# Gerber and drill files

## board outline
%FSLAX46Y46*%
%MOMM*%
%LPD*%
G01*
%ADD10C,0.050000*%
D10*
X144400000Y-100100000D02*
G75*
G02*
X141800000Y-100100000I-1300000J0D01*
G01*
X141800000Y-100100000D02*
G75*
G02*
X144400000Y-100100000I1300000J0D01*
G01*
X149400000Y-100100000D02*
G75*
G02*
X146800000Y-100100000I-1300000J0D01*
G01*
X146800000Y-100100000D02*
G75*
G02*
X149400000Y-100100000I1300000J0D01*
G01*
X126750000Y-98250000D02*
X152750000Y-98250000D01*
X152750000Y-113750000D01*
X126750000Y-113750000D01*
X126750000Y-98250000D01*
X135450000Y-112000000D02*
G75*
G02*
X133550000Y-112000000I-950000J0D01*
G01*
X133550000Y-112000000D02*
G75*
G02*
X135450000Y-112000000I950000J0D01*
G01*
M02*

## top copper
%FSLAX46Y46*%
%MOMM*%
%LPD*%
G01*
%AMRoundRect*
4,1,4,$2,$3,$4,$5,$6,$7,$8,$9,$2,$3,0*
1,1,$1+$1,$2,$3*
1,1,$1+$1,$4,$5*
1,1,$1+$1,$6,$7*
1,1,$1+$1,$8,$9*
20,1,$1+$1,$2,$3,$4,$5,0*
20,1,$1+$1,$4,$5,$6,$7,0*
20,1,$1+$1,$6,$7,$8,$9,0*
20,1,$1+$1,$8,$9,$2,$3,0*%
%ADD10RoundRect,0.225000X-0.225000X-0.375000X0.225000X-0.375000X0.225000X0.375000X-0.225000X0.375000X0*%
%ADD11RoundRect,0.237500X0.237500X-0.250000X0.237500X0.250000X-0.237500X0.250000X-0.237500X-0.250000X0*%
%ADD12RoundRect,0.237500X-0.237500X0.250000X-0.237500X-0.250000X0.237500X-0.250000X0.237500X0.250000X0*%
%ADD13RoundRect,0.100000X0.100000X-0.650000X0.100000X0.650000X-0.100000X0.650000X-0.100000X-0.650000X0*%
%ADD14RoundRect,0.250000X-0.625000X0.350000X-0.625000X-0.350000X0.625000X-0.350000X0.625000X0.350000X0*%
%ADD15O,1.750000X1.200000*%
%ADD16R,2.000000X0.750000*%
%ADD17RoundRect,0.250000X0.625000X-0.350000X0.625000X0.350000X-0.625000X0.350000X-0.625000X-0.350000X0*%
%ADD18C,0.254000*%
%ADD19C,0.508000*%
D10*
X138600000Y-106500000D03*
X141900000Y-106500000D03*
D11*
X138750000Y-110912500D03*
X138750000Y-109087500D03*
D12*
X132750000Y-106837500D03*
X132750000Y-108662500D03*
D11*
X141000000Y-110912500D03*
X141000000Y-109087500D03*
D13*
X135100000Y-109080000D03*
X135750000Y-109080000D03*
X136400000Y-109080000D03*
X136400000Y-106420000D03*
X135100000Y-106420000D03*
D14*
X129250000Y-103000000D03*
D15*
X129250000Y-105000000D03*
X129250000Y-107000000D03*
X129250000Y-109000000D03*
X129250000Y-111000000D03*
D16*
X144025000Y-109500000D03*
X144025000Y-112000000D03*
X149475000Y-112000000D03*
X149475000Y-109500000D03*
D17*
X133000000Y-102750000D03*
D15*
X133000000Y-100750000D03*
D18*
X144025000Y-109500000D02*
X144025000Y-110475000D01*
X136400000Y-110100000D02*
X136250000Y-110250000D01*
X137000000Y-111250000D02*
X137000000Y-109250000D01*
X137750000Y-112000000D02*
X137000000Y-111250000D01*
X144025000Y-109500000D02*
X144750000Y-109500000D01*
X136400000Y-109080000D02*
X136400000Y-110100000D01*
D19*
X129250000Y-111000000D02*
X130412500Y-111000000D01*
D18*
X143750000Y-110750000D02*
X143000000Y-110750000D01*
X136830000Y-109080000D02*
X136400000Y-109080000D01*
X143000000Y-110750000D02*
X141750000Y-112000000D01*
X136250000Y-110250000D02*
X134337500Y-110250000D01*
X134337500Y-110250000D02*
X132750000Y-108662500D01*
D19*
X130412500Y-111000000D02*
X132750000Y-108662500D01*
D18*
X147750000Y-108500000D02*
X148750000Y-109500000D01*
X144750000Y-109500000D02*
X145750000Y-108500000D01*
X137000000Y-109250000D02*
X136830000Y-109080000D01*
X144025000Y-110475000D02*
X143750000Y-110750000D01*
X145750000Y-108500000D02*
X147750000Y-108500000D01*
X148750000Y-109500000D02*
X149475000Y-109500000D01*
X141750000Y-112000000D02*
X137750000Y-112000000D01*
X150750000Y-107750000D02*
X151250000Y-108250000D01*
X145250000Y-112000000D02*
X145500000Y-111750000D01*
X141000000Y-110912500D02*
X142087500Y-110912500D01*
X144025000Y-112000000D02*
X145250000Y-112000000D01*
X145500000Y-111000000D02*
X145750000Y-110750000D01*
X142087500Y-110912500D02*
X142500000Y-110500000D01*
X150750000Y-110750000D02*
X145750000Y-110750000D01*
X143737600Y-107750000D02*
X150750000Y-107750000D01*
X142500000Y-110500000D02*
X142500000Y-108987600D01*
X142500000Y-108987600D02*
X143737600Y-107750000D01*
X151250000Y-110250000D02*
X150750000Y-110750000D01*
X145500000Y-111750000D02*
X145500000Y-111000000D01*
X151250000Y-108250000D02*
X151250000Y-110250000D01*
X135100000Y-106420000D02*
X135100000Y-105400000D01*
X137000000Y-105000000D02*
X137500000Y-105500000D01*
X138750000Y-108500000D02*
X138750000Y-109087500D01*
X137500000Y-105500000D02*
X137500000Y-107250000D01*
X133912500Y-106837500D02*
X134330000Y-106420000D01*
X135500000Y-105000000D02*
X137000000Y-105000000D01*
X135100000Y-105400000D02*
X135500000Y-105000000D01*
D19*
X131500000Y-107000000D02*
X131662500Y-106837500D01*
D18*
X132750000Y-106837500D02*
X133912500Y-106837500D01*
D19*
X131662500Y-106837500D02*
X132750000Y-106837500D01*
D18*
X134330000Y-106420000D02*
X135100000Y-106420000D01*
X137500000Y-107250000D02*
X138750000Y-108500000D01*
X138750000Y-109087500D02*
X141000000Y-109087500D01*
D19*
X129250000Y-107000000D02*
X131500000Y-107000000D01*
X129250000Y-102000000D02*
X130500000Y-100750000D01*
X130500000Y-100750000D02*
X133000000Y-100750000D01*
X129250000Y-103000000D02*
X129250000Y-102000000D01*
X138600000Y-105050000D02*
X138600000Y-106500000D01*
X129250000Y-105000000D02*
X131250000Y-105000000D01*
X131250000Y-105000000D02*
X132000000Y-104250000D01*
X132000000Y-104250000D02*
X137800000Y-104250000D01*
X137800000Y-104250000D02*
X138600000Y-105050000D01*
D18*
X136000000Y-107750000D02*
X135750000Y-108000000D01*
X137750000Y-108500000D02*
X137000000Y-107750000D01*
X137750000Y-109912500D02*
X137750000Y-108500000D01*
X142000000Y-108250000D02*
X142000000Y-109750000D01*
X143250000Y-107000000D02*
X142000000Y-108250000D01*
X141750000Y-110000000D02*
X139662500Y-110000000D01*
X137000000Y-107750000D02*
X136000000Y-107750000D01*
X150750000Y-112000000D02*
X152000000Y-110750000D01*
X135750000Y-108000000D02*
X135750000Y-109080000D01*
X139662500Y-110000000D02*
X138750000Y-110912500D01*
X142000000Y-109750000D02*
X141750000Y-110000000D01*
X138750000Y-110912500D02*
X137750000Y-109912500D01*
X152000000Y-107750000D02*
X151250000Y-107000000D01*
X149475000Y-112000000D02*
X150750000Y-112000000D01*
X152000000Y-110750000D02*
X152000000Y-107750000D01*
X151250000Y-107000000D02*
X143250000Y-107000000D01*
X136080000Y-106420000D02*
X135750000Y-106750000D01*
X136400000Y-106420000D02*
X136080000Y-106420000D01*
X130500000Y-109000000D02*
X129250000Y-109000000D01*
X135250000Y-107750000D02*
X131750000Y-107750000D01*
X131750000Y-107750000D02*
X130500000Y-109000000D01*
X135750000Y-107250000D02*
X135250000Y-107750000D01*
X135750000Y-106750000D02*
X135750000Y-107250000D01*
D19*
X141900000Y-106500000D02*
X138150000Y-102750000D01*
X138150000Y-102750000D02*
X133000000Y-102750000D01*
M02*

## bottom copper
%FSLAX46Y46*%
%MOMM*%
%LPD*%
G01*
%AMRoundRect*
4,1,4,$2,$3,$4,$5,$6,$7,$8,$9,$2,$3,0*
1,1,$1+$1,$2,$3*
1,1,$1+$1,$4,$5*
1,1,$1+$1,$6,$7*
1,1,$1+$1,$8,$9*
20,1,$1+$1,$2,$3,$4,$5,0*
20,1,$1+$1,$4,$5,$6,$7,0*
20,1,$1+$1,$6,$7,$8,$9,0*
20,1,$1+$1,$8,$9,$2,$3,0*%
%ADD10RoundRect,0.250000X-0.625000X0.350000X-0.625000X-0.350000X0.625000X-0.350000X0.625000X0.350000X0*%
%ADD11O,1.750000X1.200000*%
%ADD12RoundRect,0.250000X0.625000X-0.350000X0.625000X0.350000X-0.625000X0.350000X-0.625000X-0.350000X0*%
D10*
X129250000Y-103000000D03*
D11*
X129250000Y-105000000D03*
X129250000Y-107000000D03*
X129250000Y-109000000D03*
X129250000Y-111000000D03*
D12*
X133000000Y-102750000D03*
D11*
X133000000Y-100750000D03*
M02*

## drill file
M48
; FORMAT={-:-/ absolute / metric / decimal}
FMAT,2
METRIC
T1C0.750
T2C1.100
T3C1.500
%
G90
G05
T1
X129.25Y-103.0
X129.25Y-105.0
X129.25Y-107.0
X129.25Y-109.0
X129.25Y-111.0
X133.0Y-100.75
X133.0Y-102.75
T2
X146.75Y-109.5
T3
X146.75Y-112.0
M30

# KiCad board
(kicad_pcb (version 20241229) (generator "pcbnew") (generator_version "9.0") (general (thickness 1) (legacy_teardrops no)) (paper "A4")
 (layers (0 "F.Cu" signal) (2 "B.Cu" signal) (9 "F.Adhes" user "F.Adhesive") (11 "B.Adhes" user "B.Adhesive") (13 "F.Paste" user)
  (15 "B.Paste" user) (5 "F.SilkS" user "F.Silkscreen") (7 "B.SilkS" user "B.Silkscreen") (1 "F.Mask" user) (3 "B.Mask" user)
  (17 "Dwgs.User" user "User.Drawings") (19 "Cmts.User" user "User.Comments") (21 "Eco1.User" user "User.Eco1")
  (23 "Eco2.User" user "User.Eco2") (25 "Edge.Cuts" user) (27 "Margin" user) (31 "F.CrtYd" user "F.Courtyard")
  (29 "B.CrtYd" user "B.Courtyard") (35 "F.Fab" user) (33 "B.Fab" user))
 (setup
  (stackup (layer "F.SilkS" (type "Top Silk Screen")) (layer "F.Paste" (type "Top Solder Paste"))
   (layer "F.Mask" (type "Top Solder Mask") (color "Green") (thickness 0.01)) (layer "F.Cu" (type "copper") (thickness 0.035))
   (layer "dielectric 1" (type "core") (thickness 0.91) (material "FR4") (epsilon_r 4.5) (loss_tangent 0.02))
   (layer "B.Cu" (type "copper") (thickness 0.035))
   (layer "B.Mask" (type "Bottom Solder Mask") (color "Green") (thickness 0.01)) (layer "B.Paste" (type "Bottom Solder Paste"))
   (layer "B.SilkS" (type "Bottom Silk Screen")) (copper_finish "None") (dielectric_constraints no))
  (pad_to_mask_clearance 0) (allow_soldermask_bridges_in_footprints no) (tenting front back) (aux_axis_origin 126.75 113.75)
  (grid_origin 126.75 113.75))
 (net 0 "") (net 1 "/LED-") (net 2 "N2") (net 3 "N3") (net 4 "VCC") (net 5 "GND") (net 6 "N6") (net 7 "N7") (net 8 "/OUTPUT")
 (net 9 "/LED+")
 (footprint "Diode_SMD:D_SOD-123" (layer "F.Cu") (at 140.25 106.5)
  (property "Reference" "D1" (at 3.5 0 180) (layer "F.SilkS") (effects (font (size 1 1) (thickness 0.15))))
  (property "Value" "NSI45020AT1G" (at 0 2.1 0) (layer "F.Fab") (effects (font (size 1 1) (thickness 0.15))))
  (pad "1" smd roundrect (at -1.65 0) (size 0.9 1.2) (layers "F.Cu" "F.Mask" "F.Paste") (roundrect_rratio 0.25) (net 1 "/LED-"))
  (pad "2" smd roundrect (at 1.65 0) (size 0.9 1.2) (layers "F.Cu" "F.Mask" "F.Paste") (roundrect_rratio 0.25) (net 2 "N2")))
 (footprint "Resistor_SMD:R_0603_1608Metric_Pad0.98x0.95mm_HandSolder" (layer "F.Cu") (at 138.75 110 90)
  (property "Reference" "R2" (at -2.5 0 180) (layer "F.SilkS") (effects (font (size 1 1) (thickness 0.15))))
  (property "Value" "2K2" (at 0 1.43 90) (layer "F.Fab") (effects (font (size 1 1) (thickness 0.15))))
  (pad "1" smd roundrect (at -0.9125 0 90) (size 0.975 0.95) (layers "F.Cu" "F.Mask" "F.Paste") (roundrect_rratio 0.25) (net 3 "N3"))
  (pad "2" smd roundrect (at 0.9125 0 90) (size 0.975 0.95) (layers "F.Cu" "F.Mask" "F.Paste") (roundrect_rratio 0.25) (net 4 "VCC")))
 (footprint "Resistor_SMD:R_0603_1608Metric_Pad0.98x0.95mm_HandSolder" (layer "F.Cu") (at 132.75 107.75 -90)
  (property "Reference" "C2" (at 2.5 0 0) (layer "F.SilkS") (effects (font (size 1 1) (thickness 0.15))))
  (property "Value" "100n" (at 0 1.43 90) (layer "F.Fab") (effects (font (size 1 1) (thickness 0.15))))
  (pad "1" smd roundrect (at -0.9125 0 270) (size 0.975 0.95) (layers "F.Cu" "F.Mask" "F.Paste") (roundrect_rratio 0.25) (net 4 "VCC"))
  (pad "2" smd roundrect (at 0.9125 0 270) (size 0.975 0.95) (layers "F.Cu" "F.Mask" "F.Paste") (roundrect_rratio 0.25) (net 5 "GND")))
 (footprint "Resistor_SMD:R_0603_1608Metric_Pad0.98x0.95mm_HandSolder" (layer "F.Cu") (at 141 110 90)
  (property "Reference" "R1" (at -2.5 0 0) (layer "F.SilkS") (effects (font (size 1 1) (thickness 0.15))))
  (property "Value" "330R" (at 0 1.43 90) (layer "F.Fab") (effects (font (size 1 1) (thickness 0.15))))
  (pad "1" smd roundrect (at -0.9125 0 90) (size 0.975 0.95) (layers "F.Cu" "F.Mask" "F.Paste") (roundrect_rratio 0.25) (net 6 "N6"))
  (pad "2" smd roundrect (at 0.9125 0 90) (size 0.975 0.95) (layers "F.Cu" "F.Mask" "F.Paste") (roundrect_rratio 0.25) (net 4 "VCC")))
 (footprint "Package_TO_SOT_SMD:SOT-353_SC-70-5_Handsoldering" (layer "F.Cu") (at 135.75 107.75 90)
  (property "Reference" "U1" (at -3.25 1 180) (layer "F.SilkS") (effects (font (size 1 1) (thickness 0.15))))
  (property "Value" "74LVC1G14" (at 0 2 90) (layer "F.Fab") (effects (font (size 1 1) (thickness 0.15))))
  (pad "1" smd roundrect (at -1.33 -0.65 90) (size 1.5 0.4) (layers "F.Cu" "F.Mask" "F.Paste") (roundrect_rratio 0.25) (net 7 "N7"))
  (pad "2" smd roundrect (at -1.33 0 90) (size 1.5 0.4) (layers "F.Cu" "F.Mask" "F.Paste") (roundrect_rratio 0.25) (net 3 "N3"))
  (pad "3" smd roundrect (at -1.33 0.65 90) (size 1.5 0.4) (layers "F.Cu" "F.Mask" "F.Paste") (roundrect_rratio 0.25) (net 5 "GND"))
  (pad "4" smd roundrect (at 1.33 0.65 90) (size 1.5 0.4) (layers "F.Cu" "F.Mask" "F.Paste") (roundrect_rratio 0.25) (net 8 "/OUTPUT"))
  (pad "5" smd roundrect (at 1.33 -0.65 90) (size 1.5 0.4) (layers "F.Cu" "F.Mask" "F.Paste") (roundrect_rratio 0.25) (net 4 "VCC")))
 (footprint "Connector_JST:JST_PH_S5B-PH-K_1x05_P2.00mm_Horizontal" (layer "F.Cu") (at 129.25 103 -90)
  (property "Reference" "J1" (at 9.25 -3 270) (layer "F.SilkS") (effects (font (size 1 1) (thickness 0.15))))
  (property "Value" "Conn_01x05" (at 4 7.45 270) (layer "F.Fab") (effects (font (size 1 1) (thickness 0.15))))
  (pad "1" thru_hole roundrect (at 0 0 270) (size 1.2 1.75) (drill 0.75) (layers "*.Cu" "*.Mask") (remove_unused_layers no)
   (roundrect_rratio 0.208333) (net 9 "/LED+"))
  (pad "2" thru_hole oval (at 2 0 270) (size 1.2 1.75) (drill 0.75) (layers "*.Cu" "*.Mask") (remove_unused_layers no) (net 1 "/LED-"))
  (pad "3" thru_hole oval (at 4 0 270) (size 1.2 1.75) (drill 0.75) (layers "*.Cu" "*.Mask") (remove_unused_layers no) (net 4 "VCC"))
  (pad "4" thru_hole oval (at 6 0 270) (size 1.2 1.75) (drill 0.75) (layers "*.Cu" "*.Mask") (remove_unused_layers no) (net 8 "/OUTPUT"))
  (pad "5" thru_hole oval (at 8 0 270) (size 1.2 1.75) (drill 0.75) (layers "*.Cu" "*.Mask") (remove_unused_layers no) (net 5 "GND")))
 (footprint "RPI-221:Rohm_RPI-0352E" (layer "F.Cu") (at 146.75 110.75)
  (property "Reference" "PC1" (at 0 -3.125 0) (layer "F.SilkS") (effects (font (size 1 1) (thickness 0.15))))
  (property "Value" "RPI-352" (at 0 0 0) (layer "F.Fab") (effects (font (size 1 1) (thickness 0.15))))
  (pad "" np_thru_hole circle (at 0 -1.25) (size 1.1 1.1) (drill 1.1) (layers "*.Cu" "*.Mask"))
  (pad "" np_thru_hole circle (at 0 1.25) (size 1.5 1.5) (drill 1.5) (layers "*.Cu" "*.Mask"))
  (pad "1" smd rect (at -2.725 -1.25 270) (size 0.75 2) (layers "F.Cu" "F.Mask" "F.Paste") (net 5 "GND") (thermal_bridge_angle 45))
  (pad "2" smd rect (at -2.725 1.25 270) (size 0.75 2) (layers "F.Cu" "F.Mask" "F.Paste") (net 6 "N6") (thermal_bridge_angle 45))
  (pad "3" smd rect (at 2.725 1.25 270) (size 0.75 2) (layers "F.Cu" "F.Mask" "F.Paste") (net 3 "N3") (thermal_bridge_angle 45))
  (pad "4" smd rect (at 2.725 -1.25 270) (size 0.75 2) (layers "F.Cu" "F.Mask" "F.Paste") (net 5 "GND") (thermal_bridge_angle 45)))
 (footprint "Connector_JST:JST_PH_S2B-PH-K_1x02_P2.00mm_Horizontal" (layer "F.Cu") (at 133 102.75 90)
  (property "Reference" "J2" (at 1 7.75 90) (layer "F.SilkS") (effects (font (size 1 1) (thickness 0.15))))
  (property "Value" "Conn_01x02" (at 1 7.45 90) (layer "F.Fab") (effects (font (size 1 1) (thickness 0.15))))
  (pad "1" thru_hole roundrect (at 0 0 90) (size 1.2 1.75) (drill 0.75) (layers "*.Cu" "*.Mask") (remove_unused_layers no)
   (roundrect_rratio 0.208333) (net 2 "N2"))
  (pad "2" thru_hole oval (at 2 0 90) (size 1.2 1.75) (drill 0.75) (layers "*.Cu" "*.Mask") (remove_unused_layers no) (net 9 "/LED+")))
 (gr_circle (center 143.1 100.1) (end 144.4 100.1) (stroke (width 0.05) (type solid)) (fill no) (layer "Edge.Cuts"))
 (gr_circle (center 148.1 100.1) (end 149.4 100.1) (stroke (width 0.05) (type solid)) (fill no) (layer "Edge.Cuts"))
 (gr_rect (start 126.75 98.25) (end 152.75 113.75) (stroke (width 0.05) (type default)) (fill no) (layer "Edge.Cuts"))
 (gr_circle (center 134.5 112) (end 135.45 112) (stroke (width 0.05) (type solid)) (fill no) (layer "Edge.Cuts"))
 (segment (start 144.025 109.5) (end 144.025 110.475) (width 0.254) (layer "F.Cu") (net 5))
 (segment (start 136.4 110.1) (end 136.25 110.25) (width 0.254) (layer "F.Cu") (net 5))
 (segment (start 137 111.25) (end 137 109.25) (width 0.254) (layer "F.Cu") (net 5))
 (segment (start 137.75 112) (end 137 111.25) (width 0.254) (layer "F.Cu") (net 5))
 (segment (start 144.025 109.5) (end 144.75 109.5) (width 0.254) (layer "F.Cu") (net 5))
 (segment (start 136.4 109.08) (end 136.4 110.1) (width 0.254) (layer "F.Cu") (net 5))
 (segment (start 129.25 111) (end 130.4125 111) (width 0.508) (layer "F.Cu") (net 5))
 (segment (start 143.75 110.75) (end 143 110.75) (width 0.254) (layer "F.Cu") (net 5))
 (segment (start 136.83 109.08) (end 136.4 109.08) (width 0.254) (layer "F.Cu") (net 5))
 (segment (start 143 110.75) (end 141.75 112) (width 0.254) (layer "F.Cu") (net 5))
 (segment (start 136.25 110.25) (end 134.3375 110.25) (width 0.254) (layer "F.Cu") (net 5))
 (segment (start 134.3375 110.25) (end 132.75 108.6625) (width 0.254) (layer "F.Cu") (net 5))
 (segment (start 130.4125 111) (end 132.75 108.6625) (width 0.508) (layer "F.Cu") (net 5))
 (segment (start 147.75 108.5) (end 148.75 109.5) (width 0.254) (layer "F.Cu") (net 5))
 (segment (start 144.75 109.5) (end 145.75 108.5) (width 0.254) (layer "F.Cu") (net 5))
 (segment (start 137 109.25) (end 136.83 109.08) (width 0.254) (layer "F.Cu") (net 5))
 (segment (start 144.025 110.475) (end 143.75 110.75) (width 0.254) (layer "F.Cu") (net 5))
 (segment (start 145.75 108.5) (end 147.75 108.5) (width 0.254) (layer "F.Cu") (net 5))
 (segment (start 148.75 109.5) (end 149.475 109.5) (width 0.254) (layer "F.Cu") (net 5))
 (segment (start 141.75 112) (end 137.75 112) (width 0.254) (layer "F.Cu") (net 5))
 (segment (start 150.75 107.75) (end 151.25 108.25) (width 0.254) (layer "F.Cu") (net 6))
 (segment (start 145.25 112) (end 145.5 111.75) (width 0.254) (layer "F.Cu") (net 6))
 (segment (start 141 110.9125) (end 142.0875 110.9125) (width 0.254) (layer "F.Cu") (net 6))
 (segment (start 144.025 112) (end 145.25 112) (width 0.254) (layer "F.Cu") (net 6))
 (segment (start 145.5 111) (end 145.75 110.75) (width 0.254) (layer "F.Cu") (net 6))
 (segment (start 142.0875 110.9125) (end 142.5 110.5) (width 0.254) (layer "F.Cu") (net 6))
 (segment (start 150.75 110.75) (end 145.75 110.75) (width 0.254) (layer "F.Cu") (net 6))
 (segment (start 143.7376 107.75) (end 150.75 107.75) (width 0.254) (layer "F.Cu") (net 6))
 (segment (start 142.5 110.5) (end 142.5 108.9876) (width 0.254) (layer "F.Cu") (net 6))
 (segment (start 142.5 108.9876) (end 143.7376 107.75) (width 0.254) (layer "F.Cu") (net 6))
 (segment (start 151.25 110.25) (end 150.75 110.75) (width 0.254) (layer "F.Cu") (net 6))
 (segment (start 145.5 111.75) (end 145.5 111) (width 0.254) (layer "F.Cu") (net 6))
 (segment (start 151.25 108.25) (end 151.25 110.25) (width 0.254) (layer "F.Cu") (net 6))
 (segment (start 135.1 106.42) (end 135.1 105.4) (width 0.254) (layer "F.Cu") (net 4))
 (segment (start 137 105) (end 137.5 105.5) (width 0.254) (layer "F.Cu") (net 4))
 (segment (start 138.75 108.5) (end 138.75 109.0875) (width 0.254) (layer "F.Cu") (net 4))
 (segment (start 137.5 105.5) (end 137.5 107.25) (width 0.254) (layer "F.Cu") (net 4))
 (segment (start 133.9125 106.8375) (end 134.33 106.42) (width 0.254) (layer "F.Cu") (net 4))
 (segment (start 135.5 105) (end 137 105) (width 0.254) (layer "F.Cu") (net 4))
 (segment (start 135.1 105.4) (end 135.5 105) (width 0.254) (layer "F.Cu") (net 4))
 (segment (start 131.5 107) (end 131.6625 106.8375) (width 0.508) (layer "F.Cu") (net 4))
 (segment (start 132.75 106.8375) (end 133.9125 106.8375) (width 0.254) (layer "F.Cu") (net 4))
 (segment (start 131.6625 106.8375) (end 132.75 106.8375) (width 0.508) (layer "F.Cu") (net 4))
 (segment (start 134.33 106.42) (end 135.1 106.42) (width 0.254) (layer "F.Cu") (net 4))
 (segment (start 137.5 107.25) (end 138.75 108.5) (width 0.254) (layer "F.Cu") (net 4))
 (segment (start 138.75 109.0875) (end 141 109.0875) (width 0.254) (layer "F.Cu") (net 4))
 (segment (start 129.25 107) (end 131.5 107) (width 0.508) (layer "F.Cu") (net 4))
 (segment (start 129.25 102) (end 130.5 100.75) (width 0.508) (layer "F.Cu") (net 9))
 (segment (start 130.5 100.75) (end 133 100.75) (width 0.508) (layer "F.Cu") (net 9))
 (segment (start 129.25 103) (end 129.25 102) (width 0.508) (layer "F.Cu") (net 9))
 (segment (start 138.6 105.05) (end 138.6 106.5) (width 0.508) (layer "F.Cu") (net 1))
 (segment (start 129.25 105) (end 131.25 105) (width 0.508) (layer "F.Cu") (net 1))
 (segment (start 131.25 105) (end 132 104.25) (width 0.508) (layer "F.Cu") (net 1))
 (segment (start 132 104.25) (end 137.8 104.25) (width 0.508) (layer "F.Cu") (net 1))
 (segment (start 137.8 104.25) (end 138.6 105.05) (width 0.508) (layer "F.Cu") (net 1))
 (segment (start 136 107.75) (end 135.75 108) (width 0.254) (layer "F.Cu") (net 3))
 (segment (start 137.75 108.5) (end 137 107.75) (width 0.254) (layer "F.Cu") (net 3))
 (segment (start 137.75 109.9125) (end 137.75 108.5) (width 0.254) (layer "F.Cu") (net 3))
 (segment (start 142 108.25) (end 142 109.75) (width 0.254) (layer "F.Cu") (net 3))
 (segment (start 143.25 107) (end 142 108.25) (width 0.254) (layer "F.Cu") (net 3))
 (segment (start 141.75 110) (end 139.6625 110) (width 0.254) (layer "F.Cu") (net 3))
 (segment (start 137 107.75) (end 136 107.75) (width 0.254) (layer "F.Cu") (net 3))
 (segment (start 150.75 112) (end 152 110.75) (width 0.254) (layer "F.Cu") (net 3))
 (segment (start 135.75 108) (end 135.75 109.08) (width 0.254) (layer "F.Cu") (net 3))
 (segment (start 139.6625 110) (end 138.75 110.9125) (width 0.254) (layer "F.Cu") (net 3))
 (segment (start 142 109.75) (end 141.75 110) (width 0.254) (layer "F.Cu") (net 3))
 (segment (start 138.75 110.9125) (end 137.75 109.9125) (width 0.254) (layer "F.Cu") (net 3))
 (segment (start 152 107.75) (end 151.25 107) (width 0.254) (layer "F.Cu") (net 3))
 (segment (start 149.475 112) (end 150.75 112) (width 0.254) (layer "F.Cu") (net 3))
 (segment (start 152 110.75) (end 152 107.75) (width 0.254) (layer "F.Cu") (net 3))
 (segment (start 151.25 107) (end 143.25 107) (width 0.254) (layer "F.Cu") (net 3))
 (segment (start 136.08 106.42) (end 135.75 106.75) (width 0.254) (layer "F.Cu") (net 8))
 (segment (start 136.4 106.42) (end 136.08 106.42) (width 0.254) (layer "F.Cu") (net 8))
 (segment (start 130.5 109) (end 129.25 109) (width 0.254) (layer "F.Cu") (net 8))
 (segment (start 135.25 107.75) (end 131.75 107.75) (width 0.254) (layer "F.Cu") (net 8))
 (segment (start 131.75 107.75) (end 130.5 109) (width 0.254) (layer "F.Cu") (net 8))
 (segment (start 135.75 107.25) (end 135.25 107.75) (width 0.254) (layer "F.Cu") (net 8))
 (segment (start 135.75 106.75) (end 135.75 107.25) (width 0.254) (layer "F.Cu") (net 8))
 (segment (start 141.9 106.5) (end 138.15 102.75) (width 0.508) (layer "F.Cu") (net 2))
 (segment (start 138.15 102.75) (end 133 102.75) (width 0.508) (layer "F.Cu") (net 2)))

